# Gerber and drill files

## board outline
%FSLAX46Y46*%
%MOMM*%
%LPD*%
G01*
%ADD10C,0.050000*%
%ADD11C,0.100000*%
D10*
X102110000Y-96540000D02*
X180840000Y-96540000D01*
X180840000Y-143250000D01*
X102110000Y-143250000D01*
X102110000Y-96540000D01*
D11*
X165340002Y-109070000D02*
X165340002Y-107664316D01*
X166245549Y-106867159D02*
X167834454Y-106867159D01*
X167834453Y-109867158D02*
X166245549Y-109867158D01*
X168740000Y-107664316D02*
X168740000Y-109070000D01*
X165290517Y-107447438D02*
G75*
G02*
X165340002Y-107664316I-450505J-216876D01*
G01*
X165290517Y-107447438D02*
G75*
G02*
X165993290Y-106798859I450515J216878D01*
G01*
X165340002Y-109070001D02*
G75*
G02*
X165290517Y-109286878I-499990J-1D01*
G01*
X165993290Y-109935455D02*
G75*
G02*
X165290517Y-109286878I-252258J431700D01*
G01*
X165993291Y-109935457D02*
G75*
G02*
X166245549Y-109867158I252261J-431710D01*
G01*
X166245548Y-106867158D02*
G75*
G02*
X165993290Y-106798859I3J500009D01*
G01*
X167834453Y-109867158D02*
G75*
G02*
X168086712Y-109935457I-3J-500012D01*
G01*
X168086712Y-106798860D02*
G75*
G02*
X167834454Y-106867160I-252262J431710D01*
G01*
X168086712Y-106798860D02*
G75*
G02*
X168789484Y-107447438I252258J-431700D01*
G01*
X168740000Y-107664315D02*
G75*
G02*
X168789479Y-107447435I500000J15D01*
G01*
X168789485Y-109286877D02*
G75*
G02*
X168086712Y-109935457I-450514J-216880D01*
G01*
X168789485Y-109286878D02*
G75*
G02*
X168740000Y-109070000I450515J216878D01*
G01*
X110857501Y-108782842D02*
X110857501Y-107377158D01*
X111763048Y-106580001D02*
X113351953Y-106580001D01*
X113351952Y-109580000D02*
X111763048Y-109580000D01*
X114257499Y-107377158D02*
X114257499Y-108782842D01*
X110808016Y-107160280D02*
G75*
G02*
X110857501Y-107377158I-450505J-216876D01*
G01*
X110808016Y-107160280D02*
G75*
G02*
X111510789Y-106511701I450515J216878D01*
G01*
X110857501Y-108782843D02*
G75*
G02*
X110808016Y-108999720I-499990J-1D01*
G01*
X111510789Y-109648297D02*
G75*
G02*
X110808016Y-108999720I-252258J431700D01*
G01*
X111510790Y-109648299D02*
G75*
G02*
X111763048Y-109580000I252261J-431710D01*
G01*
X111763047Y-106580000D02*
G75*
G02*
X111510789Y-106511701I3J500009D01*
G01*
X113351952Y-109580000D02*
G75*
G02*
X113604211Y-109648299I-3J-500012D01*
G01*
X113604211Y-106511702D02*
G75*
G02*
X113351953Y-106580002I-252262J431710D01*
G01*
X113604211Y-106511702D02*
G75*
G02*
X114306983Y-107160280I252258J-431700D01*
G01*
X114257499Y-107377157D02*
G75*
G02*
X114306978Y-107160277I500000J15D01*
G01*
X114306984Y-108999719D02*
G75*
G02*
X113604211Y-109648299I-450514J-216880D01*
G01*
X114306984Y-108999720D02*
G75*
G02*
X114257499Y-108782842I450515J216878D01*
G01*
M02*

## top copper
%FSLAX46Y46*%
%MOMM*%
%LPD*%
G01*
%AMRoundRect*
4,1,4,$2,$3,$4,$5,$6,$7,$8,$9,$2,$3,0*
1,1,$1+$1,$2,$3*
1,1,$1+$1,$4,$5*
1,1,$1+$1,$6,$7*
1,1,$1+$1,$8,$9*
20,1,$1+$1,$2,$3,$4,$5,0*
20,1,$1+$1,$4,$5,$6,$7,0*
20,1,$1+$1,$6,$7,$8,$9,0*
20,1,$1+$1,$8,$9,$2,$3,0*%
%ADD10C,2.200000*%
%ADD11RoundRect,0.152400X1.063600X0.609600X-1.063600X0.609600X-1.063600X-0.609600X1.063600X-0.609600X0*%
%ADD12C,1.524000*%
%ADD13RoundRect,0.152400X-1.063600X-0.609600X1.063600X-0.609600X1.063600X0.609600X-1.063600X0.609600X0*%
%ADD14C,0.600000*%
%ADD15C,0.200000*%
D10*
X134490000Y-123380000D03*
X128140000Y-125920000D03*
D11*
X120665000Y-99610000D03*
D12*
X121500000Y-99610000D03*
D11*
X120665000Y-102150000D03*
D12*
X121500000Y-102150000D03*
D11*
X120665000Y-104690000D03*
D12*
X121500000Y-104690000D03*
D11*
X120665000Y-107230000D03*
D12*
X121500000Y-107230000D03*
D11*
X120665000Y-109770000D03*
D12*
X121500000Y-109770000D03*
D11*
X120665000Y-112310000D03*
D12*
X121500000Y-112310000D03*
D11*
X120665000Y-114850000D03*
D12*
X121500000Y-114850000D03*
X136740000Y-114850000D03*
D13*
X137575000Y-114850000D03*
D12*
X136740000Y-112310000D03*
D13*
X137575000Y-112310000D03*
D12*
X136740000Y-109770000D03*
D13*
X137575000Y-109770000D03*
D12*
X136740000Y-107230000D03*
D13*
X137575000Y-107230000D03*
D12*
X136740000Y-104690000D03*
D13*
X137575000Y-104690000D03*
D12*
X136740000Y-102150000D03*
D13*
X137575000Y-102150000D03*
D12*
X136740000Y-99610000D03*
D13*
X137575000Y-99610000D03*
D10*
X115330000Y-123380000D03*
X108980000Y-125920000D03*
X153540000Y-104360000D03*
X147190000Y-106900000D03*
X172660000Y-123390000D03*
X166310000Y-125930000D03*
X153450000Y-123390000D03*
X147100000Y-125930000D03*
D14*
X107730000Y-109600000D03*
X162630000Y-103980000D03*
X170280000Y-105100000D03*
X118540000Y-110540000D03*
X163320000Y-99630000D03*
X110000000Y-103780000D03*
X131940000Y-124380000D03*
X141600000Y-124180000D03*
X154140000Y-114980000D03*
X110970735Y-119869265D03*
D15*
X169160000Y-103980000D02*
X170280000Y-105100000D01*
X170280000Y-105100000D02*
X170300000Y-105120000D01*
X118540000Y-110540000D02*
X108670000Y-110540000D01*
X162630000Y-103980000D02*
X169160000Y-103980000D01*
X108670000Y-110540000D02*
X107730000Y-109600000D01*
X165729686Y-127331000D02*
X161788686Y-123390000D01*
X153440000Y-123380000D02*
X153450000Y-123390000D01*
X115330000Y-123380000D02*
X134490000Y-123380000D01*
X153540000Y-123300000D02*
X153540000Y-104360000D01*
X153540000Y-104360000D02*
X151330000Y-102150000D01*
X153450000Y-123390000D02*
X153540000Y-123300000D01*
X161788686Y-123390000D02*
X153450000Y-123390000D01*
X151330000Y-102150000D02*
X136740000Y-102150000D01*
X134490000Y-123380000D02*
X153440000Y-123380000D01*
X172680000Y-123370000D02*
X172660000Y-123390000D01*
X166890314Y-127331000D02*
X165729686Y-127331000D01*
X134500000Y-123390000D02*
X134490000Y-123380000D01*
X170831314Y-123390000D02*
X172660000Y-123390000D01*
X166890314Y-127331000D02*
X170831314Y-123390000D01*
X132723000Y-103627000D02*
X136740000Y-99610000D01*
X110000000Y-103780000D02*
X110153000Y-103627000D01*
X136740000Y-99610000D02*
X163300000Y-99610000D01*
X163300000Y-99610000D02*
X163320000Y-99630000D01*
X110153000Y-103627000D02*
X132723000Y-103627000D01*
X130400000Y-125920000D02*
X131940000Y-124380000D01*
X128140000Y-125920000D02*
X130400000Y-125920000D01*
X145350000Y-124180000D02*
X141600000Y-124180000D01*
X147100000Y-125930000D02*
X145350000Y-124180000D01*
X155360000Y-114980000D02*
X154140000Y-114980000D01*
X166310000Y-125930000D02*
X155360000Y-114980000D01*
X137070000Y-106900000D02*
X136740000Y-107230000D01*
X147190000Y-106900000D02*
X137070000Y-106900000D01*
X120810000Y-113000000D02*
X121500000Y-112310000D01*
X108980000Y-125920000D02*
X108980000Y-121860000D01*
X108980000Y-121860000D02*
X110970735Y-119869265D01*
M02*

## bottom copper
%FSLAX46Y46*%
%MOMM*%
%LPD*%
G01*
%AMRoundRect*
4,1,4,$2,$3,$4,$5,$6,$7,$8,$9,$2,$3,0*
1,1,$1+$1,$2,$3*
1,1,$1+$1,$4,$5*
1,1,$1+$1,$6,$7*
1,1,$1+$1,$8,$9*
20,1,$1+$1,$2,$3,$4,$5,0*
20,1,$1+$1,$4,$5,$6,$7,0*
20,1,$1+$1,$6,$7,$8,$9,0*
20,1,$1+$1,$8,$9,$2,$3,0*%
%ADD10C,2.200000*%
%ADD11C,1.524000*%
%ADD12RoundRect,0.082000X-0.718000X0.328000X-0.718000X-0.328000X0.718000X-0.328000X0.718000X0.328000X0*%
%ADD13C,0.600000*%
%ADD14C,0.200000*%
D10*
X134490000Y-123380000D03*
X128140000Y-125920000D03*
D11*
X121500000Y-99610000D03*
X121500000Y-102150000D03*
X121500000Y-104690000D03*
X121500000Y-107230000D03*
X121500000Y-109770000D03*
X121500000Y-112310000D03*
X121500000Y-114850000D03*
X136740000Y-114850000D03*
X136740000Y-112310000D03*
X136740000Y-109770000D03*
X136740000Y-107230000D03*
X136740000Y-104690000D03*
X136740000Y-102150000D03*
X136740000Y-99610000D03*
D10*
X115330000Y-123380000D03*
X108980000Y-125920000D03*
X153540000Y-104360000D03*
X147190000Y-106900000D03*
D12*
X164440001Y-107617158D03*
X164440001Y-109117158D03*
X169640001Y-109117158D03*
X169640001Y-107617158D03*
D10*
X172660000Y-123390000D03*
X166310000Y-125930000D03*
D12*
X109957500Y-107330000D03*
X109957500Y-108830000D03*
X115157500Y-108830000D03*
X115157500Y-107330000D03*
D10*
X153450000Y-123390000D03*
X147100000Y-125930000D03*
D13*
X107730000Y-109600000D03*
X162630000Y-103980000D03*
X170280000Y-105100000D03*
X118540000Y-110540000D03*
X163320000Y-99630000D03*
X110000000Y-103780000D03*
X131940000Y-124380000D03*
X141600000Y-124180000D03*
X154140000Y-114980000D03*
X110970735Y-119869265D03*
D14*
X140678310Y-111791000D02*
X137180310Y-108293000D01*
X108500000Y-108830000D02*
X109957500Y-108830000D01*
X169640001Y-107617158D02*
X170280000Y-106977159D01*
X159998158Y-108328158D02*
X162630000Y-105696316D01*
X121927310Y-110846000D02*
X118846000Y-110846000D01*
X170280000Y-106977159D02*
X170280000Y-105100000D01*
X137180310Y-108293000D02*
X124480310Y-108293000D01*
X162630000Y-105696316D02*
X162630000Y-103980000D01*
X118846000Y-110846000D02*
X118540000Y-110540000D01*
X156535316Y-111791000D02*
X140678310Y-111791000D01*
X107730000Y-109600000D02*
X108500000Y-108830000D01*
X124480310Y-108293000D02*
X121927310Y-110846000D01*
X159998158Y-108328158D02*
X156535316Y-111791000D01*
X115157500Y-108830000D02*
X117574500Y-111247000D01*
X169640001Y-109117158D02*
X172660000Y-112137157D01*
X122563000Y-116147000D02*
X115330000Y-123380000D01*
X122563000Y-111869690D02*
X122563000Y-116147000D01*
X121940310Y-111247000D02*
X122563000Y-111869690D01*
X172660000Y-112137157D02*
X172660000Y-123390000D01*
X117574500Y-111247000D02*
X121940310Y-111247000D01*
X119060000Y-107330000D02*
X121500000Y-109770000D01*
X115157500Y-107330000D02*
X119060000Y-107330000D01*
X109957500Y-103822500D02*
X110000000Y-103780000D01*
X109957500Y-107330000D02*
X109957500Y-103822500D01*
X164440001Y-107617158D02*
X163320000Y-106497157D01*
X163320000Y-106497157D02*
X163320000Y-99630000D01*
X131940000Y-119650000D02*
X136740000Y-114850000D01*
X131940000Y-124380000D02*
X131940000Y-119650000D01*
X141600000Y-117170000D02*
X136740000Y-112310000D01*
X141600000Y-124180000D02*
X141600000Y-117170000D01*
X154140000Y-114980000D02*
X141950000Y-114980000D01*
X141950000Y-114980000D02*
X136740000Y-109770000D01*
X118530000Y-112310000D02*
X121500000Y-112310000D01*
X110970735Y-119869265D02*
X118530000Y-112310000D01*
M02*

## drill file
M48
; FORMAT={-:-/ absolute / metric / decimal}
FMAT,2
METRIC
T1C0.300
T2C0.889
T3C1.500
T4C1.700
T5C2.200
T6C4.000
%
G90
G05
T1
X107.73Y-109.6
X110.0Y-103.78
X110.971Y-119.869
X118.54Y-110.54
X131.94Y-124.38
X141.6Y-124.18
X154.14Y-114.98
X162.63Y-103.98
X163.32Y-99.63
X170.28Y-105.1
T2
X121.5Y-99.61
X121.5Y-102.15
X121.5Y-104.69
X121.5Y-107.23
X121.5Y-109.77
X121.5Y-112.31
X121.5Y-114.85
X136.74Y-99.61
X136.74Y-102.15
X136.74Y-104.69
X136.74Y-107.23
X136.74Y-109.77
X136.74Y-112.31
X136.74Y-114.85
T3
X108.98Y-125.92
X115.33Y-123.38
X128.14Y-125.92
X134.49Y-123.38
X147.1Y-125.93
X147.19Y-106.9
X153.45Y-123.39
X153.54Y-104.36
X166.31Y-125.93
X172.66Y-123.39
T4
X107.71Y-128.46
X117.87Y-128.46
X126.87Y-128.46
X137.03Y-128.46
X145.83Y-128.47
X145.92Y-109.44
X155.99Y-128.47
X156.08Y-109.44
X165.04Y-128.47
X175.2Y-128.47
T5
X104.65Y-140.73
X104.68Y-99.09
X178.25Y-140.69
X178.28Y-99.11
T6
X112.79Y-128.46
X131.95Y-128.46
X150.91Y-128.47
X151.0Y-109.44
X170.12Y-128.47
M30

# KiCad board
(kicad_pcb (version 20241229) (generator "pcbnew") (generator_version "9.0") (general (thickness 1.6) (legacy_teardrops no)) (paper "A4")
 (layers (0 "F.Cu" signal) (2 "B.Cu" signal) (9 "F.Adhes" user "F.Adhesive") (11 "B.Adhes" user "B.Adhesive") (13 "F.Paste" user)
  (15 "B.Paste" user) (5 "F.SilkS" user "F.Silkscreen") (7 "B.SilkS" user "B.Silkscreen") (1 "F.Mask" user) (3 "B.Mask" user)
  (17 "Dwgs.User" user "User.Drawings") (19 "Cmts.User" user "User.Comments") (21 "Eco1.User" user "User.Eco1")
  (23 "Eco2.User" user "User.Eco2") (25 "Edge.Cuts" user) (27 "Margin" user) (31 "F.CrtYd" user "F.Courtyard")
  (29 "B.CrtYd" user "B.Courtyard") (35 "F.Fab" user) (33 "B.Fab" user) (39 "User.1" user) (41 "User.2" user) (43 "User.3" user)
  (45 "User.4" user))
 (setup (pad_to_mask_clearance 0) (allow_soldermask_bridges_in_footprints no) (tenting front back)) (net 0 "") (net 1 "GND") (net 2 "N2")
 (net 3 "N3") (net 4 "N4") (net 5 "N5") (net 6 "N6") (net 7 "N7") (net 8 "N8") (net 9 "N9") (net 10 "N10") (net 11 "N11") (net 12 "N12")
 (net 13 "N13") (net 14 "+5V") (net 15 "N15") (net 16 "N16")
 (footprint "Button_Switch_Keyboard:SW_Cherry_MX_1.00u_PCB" (layer "F.Cu") (at 134.49 123.38)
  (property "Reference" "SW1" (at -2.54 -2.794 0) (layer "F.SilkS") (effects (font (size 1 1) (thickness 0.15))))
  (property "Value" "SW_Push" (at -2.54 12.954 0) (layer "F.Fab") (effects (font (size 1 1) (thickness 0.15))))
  (pad "" np_thru_hole circle (at -7.62 5.08) (size 1.7 1.7) (drill 1.7) (layers "*.Cu" "*.Mask"))
  (pad "" np_thru_hole circle (at -2.54 5.08) (size 4 4) (drill 4) (layers "*.Cu" "*.Mask"))
  (pad "" np_thru_hole circle (at 2.54 5.08) (size 1.7 1.7) (drill 1.7) (layers "*.Cu" "*.Mask"))
  (pad "1" thru_hole circle (at 0 0) (size 2.2 2.2) (drill 1.5) (layers "*.Cu" "*.Mask") (remove_unused_layers no) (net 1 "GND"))
  (pad "2" thru_hole circle (at -6.35 2.54) (size 2.2 2.2) (drill 1.5) (layers "*.Cu" "*.Mask") (remove_unused_layers no) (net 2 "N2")))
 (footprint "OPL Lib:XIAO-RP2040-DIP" (layer "F.Cu") (at 129.12 107.23)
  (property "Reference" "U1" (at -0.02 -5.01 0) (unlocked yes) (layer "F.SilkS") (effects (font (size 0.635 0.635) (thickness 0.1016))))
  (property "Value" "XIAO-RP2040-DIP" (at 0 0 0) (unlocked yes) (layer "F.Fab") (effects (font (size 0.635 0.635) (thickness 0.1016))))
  (pad "1" smd roundrect (at -8.455 -7.62 180) (size 2.432 1.524) (layers "F.Cu" "F.Mask") (roundrect_rratio 0.1) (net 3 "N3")
   (thermal_bridge_angle 45))
  (pad "1" thru_hole circle (at -7.62 -7.62 180) (size 1.524 1.524) (drill 0.889) (layers "*.Cu" "*.Mask") (remove_unused_layers no)
   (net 3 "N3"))
  (pad "2" smd roundrect (at -8.455 -5.08 180) (size 2.432 1.524) (layers "F.Cu" "F.Mask") (roundrect_rratio 0.1) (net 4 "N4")
   (thermal_bridge_angle 45))
  (pad "2" thru_hole circle (at -7.62 -5.08 180) (size 1.524 1.524) (drill 0.889) (layers "*.Cu" "*.Mask") (remove_unused_layers no)
   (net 4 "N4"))
  (pad "3" smd roundrect (at -8.455 -2.54 180) (size 2.432 1.524) (layers "F.Cu" "F.Mask") (roundrect_rratio 0.1) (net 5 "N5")
   (thermal_bridge_angle 45))
  (pad "3" thru_hole circle (at -7.62 -2.54 180) (size 1.524 1.524) (drill 0.889) (layers "*.Cu" "*.Mask") (remove_unused_layers no)
   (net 5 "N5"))
  (pad "4" smd roundrect (at -8.455 0 180) (size 2.432 1.524) (layers "F.Cu" "F.Mask") (roundrect_rratio 0.1) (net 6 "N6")
   (thermal_bridge_angle 45))
  (pad "4" thru_hole circle (at -7.62 0 180) (size 1.524 1.524) (drill 0.889) (layers "*.Cu" "*.Mask") (remove_unused_layers no)
   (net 6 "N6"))
  (pad "5" smd roundrect (at -8.455 2.54 180) (size 2.432 1.524) (layers "F.Cu" "F.Mask") (roundrect_rratio 0.1) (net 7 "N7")
   (thermal_bridge_angle 45))
  (pad "5" thru_hole circle (at -7.62 2.54 180) (size 1.524 1.524) (drill 0.889) (layers "*.Cu" "*.Mask") (remove_unused_layers no)
   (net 7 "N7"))
  (pad "6" smd roundrect (at -8.455 5.08 180) (size 2.432 1.524) (layers "F.Cu" "F.Mask") (roundrect_rratio 0.1) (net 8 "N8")
   (thermal_bridge_angle 45))
  (pad "6" thru_hole circle (at -7.62 5.08 180) (size 1.524 1.524) (drill 0.889) (layers "*.Cu" "*.Mask") (remove_unused_layers no)
   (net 8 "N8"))
  (pad "7" smd roundrect (at -8.455 7.62 180) (size 2.432 1.524) (layers "F.Cu" "F.Mask") (roundrect_rratio 0.1) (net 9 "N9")
   (thermal_bridge_angle 45))
  (pad "7" thru_hole circle (at -7.62 7.62 180) (size 1.524 1.524) (drill 0.889) (layers "*.Cu" "*.Mask") (remove_unused_layers no)
   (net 9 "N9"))
  (pad "8" thru_hole circle (at 7.62 7.62) (size 1.524 1.524) (drill 0.889) (layers "*.Cu" "*.Mask") (remove_unused_layers no) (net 2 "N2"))
  (pad "8" smd roundrect (at 8.455 7.62) (size 2.432 1.524) (layers "F.Cu" "F.Mask") (roundrect_rratio 0.1) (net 2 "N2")
   (thermal_bridge_angle 45))
  (pad "9" thru_hole circle (at 7.62 5.08) (size 1.524 1.524) (drill 0.889) (layers "*.Cu" "*.Mask") (remove_unused_layers no)
   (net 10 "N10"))
  (pad "9" smd roundrect (at 8.455 5.08) (size 2.432 1.524) (layers "F.Cu" "F.Mask") (roundrect_rratio 0.1) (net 10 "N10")
   (thermal_bridge_angle 45))
  (pad "10" thru_hole circle (at 7.62 2.54) (size 1.524 1.524) (drill 0.889) (layers "*.Cu" "*.Mask") (remove_unused_layers no)
   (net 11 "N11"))
  (pad "10" smd roundrect (at 8.455 2.54) (size 2.432 1.524) (layers "F.Cu" "F.Mask") (roundrect_rratio 0.1) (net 11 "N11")
   (thermal_bridge_angle 45))
  (pad "11" thru_hole circle (at 7.62 0) (size 1.524 1.524) (drill 0.889) (layers "*.Cu" "*.Mask") (remove_unused_layers no) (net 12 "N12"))
  (pad "11" smd roundrect (at 8.455 0) (size 2.432 1.524) (layers "F.Cu" "F.Mask") (roundrect_rratio 0.1) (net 12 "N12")
   (thermal_bridge_angle 45))
  (pad "12" thru_hole circle (at 7.62 -2.54) (size 1.524 1.524) (drill 0.889) (layers "*.Cu" "*.Mask") (remove_unused_layers no)
   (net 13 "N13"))
  (pad "12" smd roundrect (at 8.455 -2.54) (size 2.432 1.524) (layers "F.Cu" "F.Mask") (roundrect_rratio 0.1) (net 13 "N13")
   (thermal_bridge_angle 45))
  (pad "13" thru_hole circle (at 7.62 -5.08) (size 1.524 1.524) (drill 0.889) (layers "*.Cu" "*.Mask") (remove_unused_layers no)
   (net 1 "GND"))
  (pad "13" smd roundrect (at 8.455 -5.08) (size 2.432 1.524) (layers "F.Cu" "F.Mask") (roundrect_rratio 0.1) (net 1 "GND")
   (thermal_bridge_angle 45))
  (pad "14" thru_hole circle (at 7.62 -7.62) (size 1.524 1.524) (drill 0.889) (layers "*.Cu" "*.Mask") (remove_unused_layers no)
   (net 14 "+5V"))
  (pad "14" smd roundrect (at 8.455 -7.62) (size 2.432 1.524) (layers "F.Cu" "F.Mask") (roundrect_rratio 0.1) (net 14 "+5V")
   (thermal_bridge_angle 45)))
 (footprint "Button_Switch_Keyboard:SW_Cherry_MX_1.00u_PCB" (layer "F.Cu") (at 115.33 123.38)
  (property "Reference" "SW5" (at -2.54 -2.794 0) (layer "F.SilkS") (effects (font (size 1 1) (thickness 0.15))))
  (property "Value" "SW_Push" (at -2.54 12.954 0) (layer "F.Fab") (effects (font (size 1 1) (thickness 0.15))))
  (pad "" np_thru_hole circle (at -7.62 5.08) (size 1.7 1.7) (drill 1.7) (layers "*.Cu" "*.Mask"))
  (pad "" np_thru_hole circle (at -2.54 5.08) (size 4 4) (drill 4) (layers "*.Cu" "*.Mask"))
  (pad "" np_thru_hole circle (at 2.54 5.08) (size 1.7 1.7) (drill 1.7) (layers "*.Cu" "*.Mask"))
  (pad "1" thru_hole circle (at 0 0) (size 2.2 2.2) (drill 1.5) (layers "*.Cu" "*.Mask") (remove_unused_layers no) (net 1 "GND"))
  (pad "2" thru_hole circle (at -6.35 2.54) (size 2.2 2.2) (drill 1.5) (layers "*.Cu" "*.Mask") (remove_unused_layers no) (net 8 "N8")))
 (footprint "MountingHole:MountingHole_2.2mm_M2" (layer "F.Cu") (at 178.28 99.11)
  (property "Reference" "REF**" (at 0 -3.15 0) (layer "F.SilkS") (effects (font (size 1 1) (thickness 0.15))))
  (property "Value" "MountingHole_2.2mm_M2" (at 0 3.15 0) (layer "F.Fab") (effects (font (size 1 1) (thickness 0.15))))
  (pad "" np_thru_hole circle (at 0 0) (size 2.2 2.2) (drill 2.2) (layers "*.Cu" "*.Mask")))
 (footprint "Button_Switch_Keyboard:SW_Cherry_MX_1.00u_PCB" (layer "F.Cu") (at 153.54 104.36)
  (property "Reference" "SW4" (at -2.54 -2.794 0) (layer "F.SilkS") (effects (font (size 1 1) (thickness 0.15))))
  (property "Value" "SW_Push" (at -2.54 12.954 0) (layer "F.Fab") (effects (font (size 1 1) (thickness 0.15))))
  (pad "" np_thru_hole circle (at -7.62 5.08) (size 1.7 1.7) (drill 1.7) (layers "*.Cu" "*.Mask"))
  (pad "" np_thru_hole circle (at -2.54 5.08) (size 4 4) (drill 4) (layers "*.Cu" "*.Mask"))
  (pad "" np_thru_hole circle (at 2.54 5.08) (size 1.7 1.7) (drill 1.7) (layers "*.Cu" "*.Mask"))
  (pad "1" thru_hole circle (at 0 0) (size 2.2 2.2) (drill 1.5) (layers "*.Cu" "*.Mask") (remove_unused_layers no) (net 1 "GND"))
  (pad "2" thru_hole circle (at -6.35 2.54) (size 2.2 2.2) (drill 1.5) (layers "*.Cu" "*.Mask") (remove_unused_layers no) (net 12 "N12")))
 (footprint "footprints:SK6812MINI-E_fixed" (layer "F.Cu") (at 167.04 108.47)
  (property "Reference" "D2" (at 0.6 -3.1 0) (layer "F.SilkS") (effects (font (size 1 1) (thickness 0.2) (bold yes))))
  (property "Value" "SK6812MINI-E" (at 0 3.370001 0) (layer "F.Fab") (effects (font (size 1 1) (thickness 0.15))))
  (fp_line (start -1.699998 0.6) (end -1.699998 -0.805684) (stroke (width 0.1) (type solid)) (layer "Edge.Cuts"))
  (fp_line (start -0.794451 -1.602841) (end 0.794454 -1.602841) (stroke (width 0.1) (type solid)) (layer "Edge.Cuts"))
  (fp_line (start 0.794453 1.397158) (end -0.794451 1.397158) (stroke (width 0.1) (type solid)) (layer "Edge.Cuts"))
  (fp_line (start 1.7 -0.805684) (end 1.7 0.6) (stroke (width 0.1) (type solid)) (layer "Edge.Cuts"))
  (fp_arc (start -1.749483 -1.022562) (mid -1.712526 -0.91691) (end -1.699998 -0.805684) (stroke (width 0.1) (type solid))
   (layer "Edge.Cuts"))
  (fp_arc (start -1.749483 -1.022562) (mid -1.63807 -1.606877) (end -1.04671 -1.671141) (stroke (width 0.1) (type solid))
   (layer "Edge.Cuts"))
  (fp_arc (start -1.699998 0.600001) (mid -1.712526 0.711226) (end -1.749483 0.816878) (stroke (width 0.1) (type solid)) (layer "Edge.Cuts"))
  (fp_arc (start -1.04671 1.465455) (mid -1.638069 1.401192) (end -1.749483 0.816878) (stroke (width 0.1) (type solid)) (layer "Edge.Cuts"))
  (fp_arc (start -1.046709 1.465457) (mid -0.925121 1.414535) (end -0.794451 1.397158) (stroke (width 0.1) (type solid)) (layer "Edge.Cuts"))
  (fp_arc (start -0.794452 -1.602842) (mid -0.925122 -1.620219) (end -1.04671 -1.671141) (stroke (width 0.1) (type solid))
   (layer "Edge.Cuts"))
  (fp_arc (start 0.794453 1.397158) (mid 0.925124 1.414535) (end 1.046712 1.465457) (stroke (width 0.1) (type solid)) (layer "Edge.Cuts"))
  (fp_arc (start 1.046712 -1.67114) (mid 0.925124 -1.620218) (end 0.794454 -1.602841) (stroke (width 0.1) (type solid)) (layer "Edge.Cuts"))
  (fp_arc (start 1.046712 -1.67114) (mid 1.638072 -1.606876) (end 1.749485 -1.022562) (stroke (width 0.1) (type solid)) (layer "Edge.Cuts"))
  (fp_arc (start 1.7 -0.805685) (mid 1.712528 -0.91691) (end 1.749485 -1.022562) (stroke (width 0.1) (type solid)) (layer "Edge.Cuts"))
  (fp_arc (start 1.749485 0.816877) (mid 1.638073 1.401193) (end 1.046712 1.465457) (stroke (width 0.1) (type solid)) (layer "Edge.Cuts"))
  (fp_arc (start 1.749485 0.816878) (mid 1.712528 0.711226) (end 1.7 0.6) (stroke (width 0.1) (type solid)) (layer "Edge.Cuts"))
  (pad "1" smd roundrect (at -2.599999 -0.852842 270) (size 0.82 1.6) (layers "B.Cu" "B.Mask" "B.Paste") (roundrect_rratio 0.1)
   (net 14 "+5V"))
  (pad "2" smd roundrect (at -2.599999 0.647158 270) (size 0.82 1.6) (layers "B.Cu" "B.Mask" "B.Paste") (roundrect_rratio 0.1)
   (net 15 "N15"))
  (pad "3" smd roundrect (at 2.600001 0.647158 270) (size 0.82 1.6) (layers "B.Cu" "B.Mask" "B.Paste") (roundrect_rratio 0.1) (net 1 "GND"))
  (pad "4" smd roundrect (at 2.600001 -0.852842 270) (size 0.82 1.6) (layers "B.Cu" "B.Mask" "B.Paste") (roundrect_rratio 0.1)
   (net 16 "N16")))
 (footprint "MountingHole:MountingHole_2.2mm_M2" (layer "F.Cu") (at 104.65 140.73)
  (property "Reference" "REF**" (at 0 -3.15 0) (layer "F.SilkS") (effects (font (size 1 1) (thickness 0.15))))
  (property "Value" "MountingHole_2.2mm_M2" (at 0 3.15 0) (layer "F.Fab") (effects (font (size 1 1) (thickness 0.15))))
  (pad "" np_thru_hole circle (at 0 0) (size 2.2 2.2) (drill 2.2) (layers "*.Cu" "*.Mask")))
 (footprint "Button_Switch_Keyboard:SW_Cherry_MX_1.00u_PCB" (layer "F.Cu") (at 172.66 123.39)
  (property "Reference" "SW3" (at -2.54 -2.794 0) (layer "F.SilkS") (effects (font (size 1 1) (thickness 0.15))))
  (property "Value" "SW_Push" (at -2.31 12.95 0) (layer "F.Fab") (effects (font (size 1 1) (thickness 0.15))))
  (pad "" np_thru_hole circle (at -7.62 5.08) (size 1.7 1.7) (drill 1.7) (layers "*.Cu" "*.Mask"))
  (pad "" np_thru_hole circle (at -2.54 5.08) (size 4 4) (drill 4) (layers "*.Cu" "*.Mask"))
  (pad "" np_thru_hole circle (at 2.54 5.08) (size 1.7 1.7) (drill 1.7) (layers "*.Cu" "*.Mask"))
  (pad "1" thru_hole circle (at 0 0) (size 2.2 2.2) (drill 1.5) (layers "*.Cu" "*.Mask") (remove_unused_layers no) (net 1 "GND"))
  (pad "2" thru_hole circle (at -6.35 2.54) (size 2.2 2.2) (drill 1.5) (layers "*.Cu" "*.Mask") (remove_unused_layers no) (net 11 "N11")))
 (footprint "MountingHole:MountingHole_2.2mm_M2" (layer "F.Cu") (at 104.68 99.09)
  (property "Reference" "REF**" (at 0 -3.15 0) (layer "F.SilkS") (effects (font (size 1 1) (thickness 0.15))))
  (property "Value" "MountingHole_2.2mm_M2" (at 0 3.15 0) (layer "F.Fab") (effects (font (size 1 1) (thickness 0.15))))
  (pad "" np_thru_hole circle (at 0 0) (size 2.2 2.2) (drill 2.2) (layers "*.Cu" "*.Mask")))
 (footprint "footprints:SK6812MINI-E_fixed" (layer "F.Cu") (at 112.557499 108.182842)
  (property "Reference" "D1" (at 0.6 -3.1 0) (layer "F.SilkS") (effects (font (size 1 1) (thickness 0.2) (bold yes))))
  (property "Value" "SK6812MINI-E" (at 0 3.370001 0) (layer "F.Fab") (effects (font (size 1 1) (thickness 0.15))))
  (fp_line (start -1.699998 0.6) (end -1.699998 -0.805684) (stroke (width 0.1) (type solid)) (layer "Edge.Cuts"))
  (fp_line (start -0.794451 -1.602841) (end 0.794454 -1.602841) (stroke (width 0.1) (type solid)) (layer "Edge.Cuts"))
  (fp_line (start 0.794453 1.397158) (end -0.794451 1.397158) (stroke (width 0.1) (type solid)) (layer "Edge.Cuts"))
  (fp_line (start 1.7 -0.805684) (end 1.7 0.6) (stroke (width 0.1) (type solid)) (layer "Edge.Cuts"))
  (fp_arc (start -1.749483 -1.022562) (mid -1.712526 -0.91691) (end -1.699998 -0.805684) (stroke (width 0.1) (type solid))
   (layer "Edge.Cuts"))
  (fp_arc (start -1.749483 -1.022562) (mid -1.63807 -1.606877) (end -1.04671 -1.671141) (stroke (width 0.1) (type solid))
   (layer "Edge.Cuts"))
  (fp_arc (start -1.699998 0.600001) (mid -1.712526 0.711226) (end -1.749483 0.816878) (stroke (width 0.1) (type solid)) (layer "Edge.Cuts"))
  (fp_arc (start -1.04671 1.465455) (mid -1.638069 1.401192) (end -1.749483 0.816878) (stroke (width 0.1) (type solid)) (layer "Edge.Cuts"))
  (fp_arc (start -1.046709 1.465457) (mid -0.925121 1.414535) (end -0.794451 1.397158) (stroke (width 0.1) (type solid)) (layer "Edge.Cuts"))
  (fp_arc (start -0.794452 -1.602842) (mid -0.925122 -1.620219) (end -1.04671 -1.671141) (stroke (width 0.1) (type solid))
   (layer "Edge.Cuts"))
  (fp_arc (start 0.794453 1.397158) (mid 0.925124 1.414535) (end 1.046712 1.465457) (stroke (width 0.1) (type solid)) (layer "Edge.Cuts"))
  (fp_arc (start 1.046712 -1.67114) (mid 0.925124 -1.620218) (end 0.794454 -1.602841) (stroke (width 0.1) (type solid)) (layer "Edge.Cuts"))
  (fp_arc (start 1.046712 -1.67114) (mid 1.638072 -1.606876) (end 1.749485 -1.022562) (stroke (width 0.1) (type solid)) (layer "Edge.Cuts"))
  (fp_arc (start 1.7 -0.805685) (mid 1.712528 -0.91691) (end 1.749485 -1.022562) (stroke (width 0.1) (type solid)) (layer "Edge.Cuts"))
  (fp_arc (start 1.749485 0.816877) (mid 1.638073 1.401193) (end 1.046712 1.465457) (stroke (width 0.1) (type solid)) (layer "Edge.Cuts"))
  (fp_arc (start 1.749485 0.816878) (mid 1.712528 0.711226) (end 1.7 0.6) (stroke (width 0.1) (type solid)) (layer "Edge.Cuts"))
  (pad "1" smd roundrect (at -2.599999 -0.852842 270) (size 0.82 1.6) (layers "B.Cu" "B.Mask" "B.Paste") (roundrect_rratio 0.1)
   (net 14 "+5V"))
  (pad "2" smd roundrect (at -2.599999 0.647158 270) (size 0.82 1.6) (layers "B.Cu" "B.Mask" "B.Paste") (roundrect_rratio 0.1)
   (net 16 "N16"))
  (pad "3" smd roundrect (at 2.600001 0.647158 270) (size 0.82 1.6) (layers "B.Cu" "B.Mask" "B.Paste") (roundrect_rratio 0.1) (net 1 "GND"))
  (pad "4" smd roundrect (at 2.600001 -0.852842 270) (size 0.82 1.6) (layers "B.Cu" "B.Mask" "B.Paste") (roundrect_rratio 0.1) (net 7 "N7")))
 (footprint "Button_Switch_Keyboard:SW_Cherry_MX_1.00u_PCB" (layer "F.Cu") (at 153.45 123.39)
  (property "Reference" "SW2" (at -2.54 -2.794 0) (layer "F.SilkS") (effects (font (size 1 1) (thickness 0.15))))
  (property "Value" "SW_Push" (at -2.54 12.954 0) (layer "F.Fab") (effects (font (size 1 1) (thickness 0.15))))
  (pad "" np_thru_hole circle (at -7.62 5.08) (size 1.7 1.7) (drill 1.7) (layers "*.Cu" "*.Mask"))
  (pad "" np_thru_hole circle (at -2.54 5.08) (size 4 4) (drill 4) (layers "*.Cu" "*.Mask"))
  (pad "" np_thru_hole circle (at 2.54 5.08) (size 1.7 1.7) (drill 1.7) (layers "*.Cu" "*.Mask"))
  (pad "1" thru_hole circle (at 0 0) (size 2.2 2.2) (drill 1.5) (layers "*.Cu" "*.Mask") (remove_unused_layers no) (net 1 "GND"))
  (pad "2" thru_hole circle (at -6.35 2.54) (size 2.2 2.2) (drill 1.5) (layers "*.Cu" "*.Mask") (remove_unused_layers no) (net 10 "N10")))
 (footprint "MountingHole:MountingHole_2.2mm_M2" (layer "F.Cu") (at 178.25 140.69)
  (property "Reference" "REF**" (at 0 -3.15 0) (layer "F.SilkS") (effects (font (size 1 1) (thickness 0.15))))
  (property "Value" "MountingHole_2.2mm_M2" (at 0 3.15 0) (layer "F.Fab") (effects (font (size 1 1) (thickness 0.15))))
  (pad "" np_thru_hole circle (at 0 0) (size 2.2 2.2) (drill 2.2) (layers "*.Cu" "*.Mask")))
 (gr_rect (start 102.11 96.54) (end 180.84 143.25) (stroke (width 0.05) (type default)) (fill no) (layer "Edge.Cuts"))
 (segment (start 169.16 103.98) (end 170.28 105.1) (width 0.2) (layer "F.Cu") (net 16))
 (segment (start 170.28 105.1) (end 170.3 105.12) (width 0.2) (layer "F.Cu") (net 16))
 (segment (start 118.54 110.54) (end 108.67 110.54) (width 0.2) (layer "F.Cu") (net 16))
 (segment (start 162.63 103.98) (end 169.16 103.98) (width 0.2) (layer "F.Cu") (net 16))
 (segment (start 108.67 110.54) (end 107.73 109.6) (width 0.2) (layer "F.Cu") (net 16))
 (via (at 107.73 109.6) (size 0.6) (drill 0.3) (layers "F.Cu" "B.Cu") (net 16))
 (via (at 162.63 103.98) (size 0.6) (drill 0.3) (layers "F.Cu" "B.Cu") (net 16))
 (via (at 170.28 105.1) (size 0.6) (drill 0.3) (layers "F.Cu" "B.Cu") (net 16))
 (via (at 118.54 110.54) (size 0.6) (drill 0.3) (layers "F.Cu" "B.Cu") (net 16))
 (segment (start 140.67831 111.791) (end 137.18031 108.293) (width 0.2) (layer "B.Cu") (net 16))
 (segment (start 108.5 108.83) (end 109.9575 108.83) (width 0.2) (layer "B.Cu") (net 16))
 (segment (start 169.640001 107.617158) (end 170.28 106.977159) (width 0.2) (layer "B.Cu") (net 16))
 (segment (start 159.998158 108.328158) (end 162.63 105.696316) (width 0.2) (layer "B.Cu") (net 16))
 (segment (start 121.92731 110.846) (end 118.846 110.846) (width 0.2) (layer "B.Cu") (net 16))
 (segment (start 170.28 106.977159) (end 170.28 105.1) (width 0.2) (layer "B.Cu") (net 16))
 (segment (start 137.18031 108.293) (end 124.48031 108.293) (width 0.2) (layer "B.Cu") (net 16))
 (segment (start 162.63 105.696316) (end 162.63 103.98) (width 0.2) (layer "B.Cu") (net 16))
 (segment (start 118.846 110.846) (end 118.54 110.54) (width 0.2) (layer "B.Cu") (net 16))
 (segment (start 156.535316 111.791) (end 140.67831 111.791) (width 0.2) (layer "B.Cu") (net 16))
 (segment (start 107.73 109.6) (end 108.5 108.83) (width 0.2) (layer "B.Cu") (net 16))
 (segment (start 124.48031 108.293) (end 121.92731 110.846) (width 0.2) (layer "B.Cu") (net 16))
 (segment (start 159.998158 108.328158) (end 156.535316 111.791) (width 0.2) (layer "B.Cu") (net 16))
 (segment (start 165.729686 127.331) (end 161.788686 123.39) (width 0.2) (layer "F.Cu") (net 1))
 (segment (start 153.44 123.38) (end 153.45 123.39) (width 0.2) (layer "F.Cu") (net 1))
 (segment (start 115.33 123.38) (end 134.49 123.38) (width 0.2) (layer "F.Cu") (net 1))
 (segment (start 153.54 123.3) (end 153.54 104.36) (width 0.2) (layer "F.Cu") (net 1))
 (segment (start 153.54 104.36) (end 151.33 102.15) (width 0.2) (layer "F.Cu") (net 1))
 (segment (start 153.45 123.39) (end 153.54 123.3) (width 0.2) (layer "F.Cu") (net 1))
 (segment (start 161.788686 123.39) (end 153.45 123.39) (width 0.2) (layer "F.Cu") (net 1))
 (segment (start 151.33 102.15) (end 136.74 102.15) (width 0.2) (layer "F.Cu") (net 1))
 (segment (start 134.49 123.38) (end 153.44 123.38) (width 0.2) (layer "F.Cu") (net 1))
 (segment (start 172.68 123.37) (end 172.66 123.39) (width 0.2) (layer "F.Cu") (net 1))
 (segment (start 166.890314 127.331) (end 165.729686 127.331) (width 0.2) (layer "F.Cu") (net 1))
 (segment (start 134.5 123.39) (end 134.49 123.38) (width 0.2) (layer "F.Cu") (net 1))
 (segment (start 170.831314 123.39) (end 172.66 123.39) (width 0.2) (layer "F.Cu") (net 1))
 (segment (start 166.890314 127.331) (end 170.831314 123.39) (width 0.2) (layer "F.Cu") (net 1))
 (segment (start 115.1575 108.83) (end 117.5745 111.247) (width 0.2) (layer "B.Cu") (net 1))
 (segment (start 169.640001 109.117158) (end 172.66 112.137157) (width 0.2) (layer "B.Cu") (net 1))
 (segment (start 122.563 116.147) (end 115.33 123.38) (width 0.2) (layer "B.Cu") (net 1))
 (segment (start 122.563 111.86969) (end 122.563 116.147) (width 0.2) (layer "B.Cu") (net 1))
 (segment (start 121.94031 111.247) (end 122.563 111.86969) (width 0.2) (layer "B.Cu") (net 1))
 (segment (start 172.66 112.137157) (end 172.66 123.39) (width 0.2) (layer "B.Cu") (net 1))
 (segment (start 117.5745 111.247) (end 121.94031 111.247) (width 0.2) (layer "B.Cu") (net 1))
 (segment (start 119.06 107.33) (end 121.5 109.77) (width 0.2) (layer "B.Cu") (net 7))
 (segment (start 115.1575 107.33) (end 119.06 107.33) (width 0.2) (layer "B.Cu") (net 7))
 (segment (start 132.723 103.627) (end 136.74 99.61) (width 0.2) (layer "F.Cu") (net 14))
 (segment (start 110 103.78) (end 110.153 103.627) (width 0.2) (layer "F.Cu") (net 14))
 (segment (start 136.74 99.61) (end 163.3 99.61) (width 0.2) (layer "F.Cu") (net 14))
 (segment (start 163.3 99.61) (end 163.32 99.63) (width 0.2) (layer "F.Cu") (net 14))
 (segment (start 110.153 103.627) (end 132.723 103.627) (width 0.2) (layer "F.Cu") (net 14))
 (via (at 163.32 99.63) (size 0.6) (drill 0.3) (layers "F.Cu" "B.Cu") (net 14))
 (via (at 110 103.78) (size 0.6) (drill 0.3) (layers "F.Cu" "B.Cu") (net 14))
 (segment (start 109.9575 103.8225) (end 110 103.78) (width 0.2) (layer "B.Cu") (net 14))
 (segment (start 109.9575 107.33) (end 109.9575 103.8225) (width 0.2) (layer "B.Cu") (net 14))
 (segment (start 164.440001 107.617158) (end 163.32 106.497157) (width 0.2) (layer "B.Cu") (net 14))
 (segment (start 163.32 106.497157) (end 163.32 99.63) (width 0.2) (layer "B.Cu") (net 14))
 (segment (start 130.4 125.92) (end 131.94 124.38) (width 0.2) (layer "F.Cu") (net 2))
 (segment (start 128.14 125.92) (end 130.4 125.92) (width 0.2) (layer "F.Cu") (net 2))
 (via (at 131.94 124.38) (size 0.6) (drill 0.3) (layers "F.Cu" "B.Cu") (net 2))
 (segment (start 131.94 119.65) (end 136.74 114.85) (width 0.2) (layer "B.Cu") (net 2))
 (segment (start 131.94 124.38) (end 131.94 119.65) (width 0.2) (layer "B.Cu") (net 2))
 (segment (start 145.35 124.18) (end 141.6 124.18) (width 0.2) (layer "F.Cu") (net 10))
 (segment (start 147.1 125.93) (end 145.35 124.18) (width 0.2) (layer "F.Cu") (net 10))
 (via (at 141.6 124.18) (size 0.6) (drill 0.3) (layers "F.Cu" "B.Cu") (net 10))
 (segment (start 141.6 117.17) (end 136.74 112.31) (width 0.2) (layer "B.Cu") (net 10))
 (segment (start 141.6 124.18) (end 141.6 117.17) (width 0.2) (layer "B.Cu") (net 10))
 (segment (start 155.36 114.98) (end 154.14 114.98) (width 0.2) (layer "F.Cu") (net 11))
 (segment (start 166.31 125.93) (end 155.36 114.98) (width 0.2) (layer "F.Cu") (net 11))
 (via (at 154.14 114.98) (size 0.6) (drill 0.3) (layers "F.Cu" "B.Cu") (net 11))
 (segment (start 154.14 114.98) (end 141.95 114.98) (width 0.2) (layer "B.Cu") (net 11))
 (segment (start 141.95 114.98) (end 136.74 109.77) (width 0.2) (layer "B.Cu") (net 11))
 (segment (start 137.07 106.9) (end 136.74 107.23) (width 0.2) (layer "F.Cu") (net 12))
 (segment (start 147.19 106.9) (end 137.07 106.9) (width 0.2) (layer "F.Cu") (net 12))
 (segment (start 120.81 113) (end 121.5 112.31) (width 0.2) (layer "F.Cu") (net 8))
 (segment (start 108.98 125.92) (end 108.98 121.86) (width 0.2) (layer "F.Cu") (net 8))
 (segment (start 108.98 121.86) (end 110.970735 119.869265) (width 0.2) (layer "F.Cu") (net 8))
 (via (at 110.970735 119.869265) (size 0.6) (drill 0.3) (layers "F.Cu" "B.Cu") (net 8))
 (segment (start 118.53 112.31) (end 121.5 112.31) (width 0.2) (layer "B.Cu") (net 8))
 (segment (start 110.970735 119.869265) (end 118.53 112.31) (width 0.2) (layer "B.Cu") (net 8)))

